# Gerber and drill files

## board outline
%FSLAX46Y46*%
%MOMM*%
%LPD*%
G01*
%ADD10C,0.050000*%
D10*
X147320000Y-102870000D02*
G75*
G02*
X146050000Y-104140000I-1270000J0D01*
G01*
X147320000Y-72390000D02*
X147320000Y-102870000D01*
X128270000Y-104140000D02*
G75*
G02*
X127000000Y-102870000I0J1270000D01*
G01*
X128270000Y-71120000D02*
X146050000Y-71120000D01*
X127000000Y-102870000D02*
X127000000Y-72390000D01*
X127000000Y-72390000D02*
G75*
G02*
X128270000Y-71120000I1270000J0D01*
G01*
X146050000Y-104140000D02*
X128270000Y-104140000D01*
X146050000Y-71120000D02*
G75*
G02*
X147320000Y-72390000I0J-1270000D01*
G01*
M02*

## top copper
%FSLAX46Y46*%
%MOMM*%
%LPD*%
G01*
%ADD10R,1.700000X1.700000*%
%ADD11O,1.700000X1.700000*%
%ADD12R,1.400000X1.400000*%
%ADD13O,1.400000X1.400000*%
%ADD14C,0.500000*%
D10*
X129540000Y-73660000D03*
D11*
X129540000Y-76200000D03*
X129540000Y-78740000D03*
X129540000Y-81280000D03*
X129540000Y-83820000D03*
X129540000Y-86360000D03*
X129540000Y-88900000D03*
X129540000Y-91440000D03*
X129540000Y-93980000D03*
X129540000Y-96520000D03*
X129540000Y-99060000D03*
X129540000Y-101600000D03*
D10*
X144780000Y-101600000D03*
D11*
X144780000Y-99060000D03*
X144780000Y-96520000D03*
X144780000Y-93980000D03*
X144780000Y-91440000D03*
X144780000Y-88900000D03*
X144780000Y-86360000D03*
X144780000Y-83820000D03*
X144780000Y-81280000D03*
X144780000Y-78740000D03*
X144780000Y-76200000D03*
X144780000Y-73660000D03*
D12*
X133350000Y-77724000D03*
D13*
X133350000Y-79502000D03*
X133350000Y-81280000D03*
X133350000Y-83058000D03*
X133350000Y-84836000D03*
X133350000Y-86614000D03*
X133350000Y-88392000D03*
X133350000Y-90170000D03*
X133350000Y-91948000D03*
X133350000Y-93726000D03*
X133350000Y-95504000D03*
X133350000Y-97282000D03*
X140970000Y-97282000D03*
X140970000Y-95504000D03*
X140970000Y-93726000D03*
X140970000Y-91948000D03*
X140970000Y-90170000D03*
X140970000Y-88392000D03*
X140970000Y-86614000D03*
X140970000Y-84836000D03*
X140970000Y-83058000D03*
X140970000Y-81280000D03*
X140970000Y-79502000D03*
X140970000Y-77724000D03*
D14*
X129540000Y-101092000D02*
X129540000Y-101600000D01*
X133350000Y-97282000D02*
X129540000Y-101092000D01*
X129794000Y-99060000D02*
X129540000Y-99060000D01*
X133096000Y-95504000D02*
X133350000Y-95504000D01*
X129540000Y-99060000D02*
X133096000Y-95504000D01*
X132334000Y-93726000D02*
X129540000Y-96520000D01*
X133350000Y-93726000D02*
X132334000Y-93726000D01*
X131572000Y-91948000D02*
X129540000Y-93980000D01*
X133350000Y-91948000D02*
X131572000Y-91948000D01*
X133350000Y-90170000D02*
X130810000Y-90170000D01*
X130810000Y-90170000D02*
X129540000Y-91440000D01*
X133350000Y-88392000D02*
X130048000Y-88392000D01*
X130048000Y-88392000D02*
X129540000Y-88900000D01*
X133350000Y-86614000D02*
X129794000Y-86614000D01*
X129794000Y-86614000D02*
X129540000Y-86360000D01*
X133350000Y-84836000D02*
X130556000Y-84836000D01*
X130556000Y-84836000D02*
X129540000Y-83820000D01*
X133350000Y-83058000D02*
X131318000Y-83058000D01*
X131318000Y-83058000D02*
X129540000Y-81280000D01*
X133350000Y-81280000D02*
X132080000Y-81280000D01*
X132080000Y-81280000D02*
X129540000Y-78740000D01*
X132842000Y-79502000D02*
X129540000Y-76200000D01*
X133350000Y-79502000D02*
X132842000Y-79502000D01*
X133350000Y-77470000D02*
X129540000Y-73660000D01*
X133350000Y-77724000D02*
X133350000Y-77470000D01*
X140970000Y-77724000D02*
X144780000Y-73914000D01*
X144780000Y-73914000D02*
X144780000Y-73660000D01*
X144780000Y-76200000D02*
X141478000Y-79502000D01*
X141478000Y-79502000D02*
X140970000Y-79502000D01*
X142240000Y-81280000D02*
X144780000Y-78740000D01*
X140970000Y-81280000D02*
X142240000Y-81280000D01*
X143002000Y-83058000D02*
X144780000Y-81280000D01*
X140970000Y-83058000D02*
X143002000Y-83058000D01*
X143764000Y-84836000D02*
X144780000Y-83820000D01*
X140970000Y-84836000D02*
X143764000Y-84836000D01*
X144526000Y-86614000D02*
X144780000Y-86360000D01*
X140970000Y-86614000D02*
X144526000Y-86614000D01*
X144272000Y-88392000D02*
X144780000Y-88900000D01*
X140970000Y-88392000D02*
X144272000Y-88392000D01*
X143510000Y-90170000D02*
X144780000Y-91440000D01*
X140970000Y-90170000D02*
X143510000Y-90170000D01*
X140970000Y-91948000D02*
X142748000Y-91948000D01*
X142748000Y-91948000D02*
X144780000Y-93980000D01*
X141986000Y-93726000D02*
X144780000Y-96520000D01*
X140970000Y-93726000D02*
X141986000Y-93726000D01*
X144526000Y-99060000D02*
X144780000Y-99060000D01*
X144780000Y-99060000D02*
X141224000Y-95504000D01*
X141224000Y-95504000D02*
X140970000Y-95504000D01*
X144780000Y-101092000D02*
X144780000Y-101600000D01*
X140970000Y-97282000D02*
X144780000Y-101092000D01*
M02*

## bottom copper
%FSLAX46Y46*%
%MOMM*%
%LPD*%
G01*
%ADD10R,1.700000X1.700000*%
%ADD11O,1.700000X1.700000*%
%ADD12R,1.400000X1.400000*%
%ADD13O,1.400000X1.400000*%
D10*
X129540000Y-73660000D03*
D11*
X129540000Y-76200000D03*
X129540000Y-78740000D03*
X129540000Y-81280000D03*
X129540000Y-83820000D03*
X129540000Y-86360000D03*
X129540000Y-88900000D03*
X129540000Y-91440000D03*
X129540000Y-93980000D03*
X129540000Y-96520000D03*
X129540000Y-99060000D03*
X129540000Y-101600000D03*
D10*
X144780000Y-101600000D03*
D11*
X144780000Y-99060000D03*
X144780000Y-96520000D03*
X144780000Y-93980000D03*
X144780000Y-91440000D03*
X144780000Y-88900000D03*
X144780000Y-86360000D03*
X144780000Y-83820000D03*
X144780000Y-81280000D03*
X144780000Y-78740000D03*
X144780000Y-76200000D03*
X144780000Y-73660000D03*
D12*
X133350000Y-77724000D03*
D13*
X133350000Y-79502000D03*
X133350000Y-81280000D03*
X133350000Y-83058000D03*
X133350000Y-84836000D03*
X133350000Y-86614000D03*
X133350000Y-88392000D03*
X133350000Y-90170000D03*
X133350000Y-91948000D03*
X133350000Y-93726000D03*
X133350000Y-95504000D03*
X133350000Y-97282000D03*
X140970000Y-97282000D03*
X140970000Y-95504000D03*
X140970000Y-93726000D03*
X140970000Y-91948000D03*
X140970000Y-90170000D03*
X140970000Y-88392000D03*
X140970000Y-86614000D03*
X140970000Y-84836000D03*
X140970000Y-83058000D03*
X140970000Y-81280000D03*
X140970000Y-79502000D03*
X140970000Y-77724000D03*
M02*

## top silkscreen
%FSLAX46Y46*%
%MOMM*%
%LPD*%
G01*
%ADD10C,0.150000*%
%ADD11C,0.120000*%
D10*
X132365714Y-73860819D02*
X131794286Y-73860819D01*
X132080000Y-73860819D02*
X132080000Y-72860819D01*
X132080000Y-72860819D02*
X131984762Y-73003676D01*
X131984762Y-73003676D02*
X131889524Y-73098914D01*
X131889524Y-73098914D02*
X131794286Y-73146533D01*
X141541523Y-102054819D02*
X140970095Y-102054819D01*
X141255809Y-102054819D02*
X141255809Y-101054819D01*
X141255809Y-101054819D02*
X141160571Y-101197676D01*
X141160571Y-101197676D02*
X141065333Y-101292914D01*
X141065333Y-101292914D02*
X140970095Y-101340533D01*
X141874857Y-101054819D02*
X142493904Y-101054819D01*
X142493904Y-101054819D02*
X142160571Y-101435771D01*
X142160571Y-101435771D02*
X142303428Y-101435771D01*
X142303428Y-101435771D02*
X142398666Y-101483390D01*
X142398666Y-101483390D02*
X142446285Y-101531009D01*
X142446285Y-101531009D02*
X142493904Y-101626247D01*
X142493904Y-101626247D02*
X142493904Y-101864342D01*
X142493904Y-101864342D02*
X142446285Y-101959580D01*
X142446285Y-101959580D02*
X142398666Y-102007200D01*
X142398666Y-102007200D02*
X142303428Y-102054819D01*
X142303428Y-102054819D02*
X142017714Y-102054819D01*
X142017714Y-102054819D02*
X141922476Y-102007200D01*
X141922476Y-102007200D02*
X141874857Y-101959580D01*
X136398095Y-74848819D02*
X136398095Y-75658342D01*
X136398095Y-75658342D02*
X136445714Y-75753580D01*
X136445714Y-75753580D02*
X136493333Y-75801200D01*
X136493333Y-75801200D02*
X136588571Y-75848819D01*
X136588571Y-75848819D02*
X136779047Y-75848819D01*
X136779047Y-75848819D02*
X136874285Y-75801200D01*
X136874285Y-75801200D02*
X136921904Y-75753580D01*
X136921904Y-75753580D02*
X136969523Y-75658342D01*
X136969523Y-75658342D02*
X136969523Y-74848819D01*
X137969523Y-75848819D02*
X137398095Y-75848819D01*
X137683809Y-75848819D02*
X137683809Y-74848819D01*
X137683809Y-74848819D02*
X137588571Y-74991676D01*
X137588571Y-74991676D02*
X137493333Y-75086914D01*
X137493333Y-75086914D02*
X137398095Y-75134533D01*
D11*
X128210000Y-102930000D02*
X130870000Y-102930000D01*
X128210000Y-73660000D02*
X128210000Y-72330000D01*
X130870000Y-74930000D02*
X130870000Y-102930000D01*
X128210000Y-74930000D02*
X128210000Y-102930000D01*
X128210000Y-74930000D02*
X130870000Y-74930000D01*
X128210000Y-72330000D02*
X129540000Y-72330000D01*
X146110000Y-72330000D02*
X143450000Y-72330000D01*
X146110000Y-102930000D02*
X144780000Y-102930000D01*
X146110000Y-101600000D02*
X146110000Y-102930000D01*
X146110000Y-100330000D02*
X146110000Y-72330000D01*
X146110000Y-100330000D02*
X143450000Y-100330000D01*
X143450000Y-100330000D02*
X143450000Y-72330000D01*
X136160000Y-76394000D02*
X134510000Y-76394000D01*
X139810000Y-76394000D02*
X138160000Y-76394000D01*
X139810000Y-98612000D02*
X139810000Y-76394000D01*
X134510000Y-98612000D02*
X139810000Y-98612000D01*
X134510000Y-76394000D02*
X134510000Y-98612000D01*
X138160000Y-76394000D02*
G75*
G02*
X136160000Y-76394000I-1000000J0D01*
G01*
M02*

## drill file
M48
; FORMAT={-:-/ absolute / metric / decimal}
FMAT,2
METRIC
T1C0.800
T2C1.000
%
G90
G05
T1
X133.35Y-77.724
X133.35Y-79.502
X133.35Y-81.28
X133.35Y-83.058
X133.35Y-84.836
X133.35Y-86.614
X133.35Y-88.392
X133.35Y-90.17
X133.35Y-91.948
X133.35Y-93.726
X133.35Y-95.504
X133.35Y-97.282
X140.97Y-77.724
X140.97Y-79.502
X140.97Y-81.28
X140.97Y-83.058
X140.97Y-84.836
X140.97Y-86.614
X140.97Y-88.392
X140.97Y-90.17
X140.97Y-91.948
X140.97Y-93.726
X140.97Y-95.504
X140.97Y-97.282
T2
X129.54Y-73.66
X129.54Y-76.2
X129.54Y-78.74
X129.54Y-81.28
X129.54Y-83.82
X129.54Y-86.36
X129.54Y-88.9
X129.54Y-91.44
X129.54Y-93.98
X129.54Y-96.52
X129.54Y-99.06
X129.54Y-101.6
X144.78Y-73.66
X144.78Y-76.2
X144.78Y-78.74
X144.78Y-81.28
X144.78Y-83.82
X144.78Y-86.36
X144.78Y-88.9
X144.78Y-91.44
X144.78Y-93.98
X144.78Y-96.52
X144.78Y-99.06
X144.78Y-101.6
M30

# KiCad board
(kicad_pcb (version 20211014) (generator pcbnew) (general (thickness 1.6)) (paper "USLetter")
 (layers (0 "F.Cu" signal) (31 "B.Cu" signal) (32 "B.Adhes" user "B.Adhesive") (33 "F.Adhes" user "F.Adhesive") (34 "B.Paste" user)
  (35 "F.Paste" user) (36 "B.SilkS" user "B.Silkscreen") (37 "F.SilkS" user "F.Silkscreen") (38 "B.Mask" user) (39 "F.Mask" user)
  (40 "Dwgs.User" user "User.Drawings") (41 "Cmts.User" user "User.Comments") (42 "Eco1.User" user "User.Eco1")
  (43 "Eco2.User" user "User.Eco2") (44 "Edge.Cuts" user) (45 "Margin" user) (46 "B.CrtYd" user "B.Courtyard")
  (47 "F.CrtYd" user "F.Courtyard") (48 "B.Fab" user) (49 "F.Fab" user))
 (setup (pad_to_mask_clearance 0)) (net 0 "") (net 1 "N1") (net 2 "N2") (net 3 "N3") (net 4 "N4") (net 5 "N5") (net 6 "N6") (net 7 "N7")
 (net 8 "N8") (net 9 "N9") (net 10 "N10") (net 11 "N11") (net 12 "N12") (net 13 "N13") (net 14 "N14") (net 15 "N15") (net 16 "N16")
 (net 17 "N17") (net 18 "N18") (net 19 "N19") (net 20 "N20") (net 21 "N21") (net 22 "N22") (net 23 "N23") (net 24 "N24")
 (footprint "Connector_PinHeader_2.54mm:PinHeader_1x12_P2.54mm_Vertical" (layer "F.Cu") (at 129.54 73.66)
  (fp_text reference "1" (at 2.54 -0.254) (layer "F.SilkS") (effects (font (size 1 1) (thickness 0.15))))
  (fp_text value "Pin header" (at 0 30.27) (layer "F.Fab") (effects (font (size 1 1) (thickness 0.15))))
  (fp_line (start -1.33 29.27) (end 1.33 29.27) (layer "F.SilkS") (width 0.12))
  (fp_line (start -1.33 0) (end -1.33 -1.33) (layer "F.SilkS") (width 0.12))
  (fp_line (start 1.33 1.27) (end 1.33 29.27) (layer "F.SilkS") (width 0.12))
  (fp_line (start -1.33 1.27) (end -1.33 29.27) (layer "F.SilkS") (width 0.12))
  (fp_line (start -1.33 1.27) (end 1.33 1.27) (layer "F.SilkS") (width 0.12))
  (fp_line (start -1.33 -1.33) (end 0 -1.33) (layer "F.SilkS") (width 0.12))
  (pad "1" thru_hole rect locked (at 0 0) (size 1.7 1.7) (drill 1) (layers *.Cu *.Mask) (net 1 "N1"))
  (pad "2" thru_hole oval locked (at 0 2.54) (size 1.7 1.7) (drill 1) (layers *.Cu *.Mask) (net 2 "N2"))
  (pad "3" thru_hole oval locked (at 0 5.08) (size 1.7 1.7) (drill 1) (layers *.Cu *.Mask) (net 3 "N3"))
  (pad "4" thru_hole oval locked (at 0 7.62) (size 1.7 1.7) (drill 1) (layers *.Cu *.Mask) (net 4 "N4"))
  (pad "5" thru_hole oval locked (at 0 10.16) (size 1.7 1.7) (drill 1) (layers *.Cu *.Mask) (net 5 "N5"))
  (pad "6" thru_hole oval locked (at 0 12.7) (size 1.7 1.7) (drill 1) (layers *.Cu *.Mask) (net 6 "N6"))
  (pad "7" thru_hole oval locked (at 0 15.24) (size 1.7 1.7) (drill 1) (layers *.Cu *.Mask) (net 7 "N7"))
  (pad "8" thru_hole oval locked (at 0 17.78) (size 1.7 1.7) (drill 1) (layers *.Cu *.Mask) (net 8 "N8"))
  (pad "9" thru_hole oval locked (at 0 20.32) (size 1.7 1.7) (drill 1) (layers *.Cu *.Mask) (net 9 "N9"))
  (pad "10" thru_hole oval locked (at 0 22.86) (size 1.7 1.7) (drill 1) (layers *.Cu *.Mask) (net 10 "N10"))
  (pad "11" thru_hole oval locked (at 0 25.4) (size 1.7 1.7) (drill 1) (layers *.Cu *.Mask) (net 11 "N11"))
  (pad "12" thru_hole oval locked (at 0 27.94) (size 1.7 1.7) (drill 1) (layers *.Cu *.Mask) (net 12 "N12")))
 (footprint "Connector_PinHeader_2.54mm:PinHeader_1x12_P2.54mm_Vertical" (layer "F.Cu") (at 144.78 101.6 180)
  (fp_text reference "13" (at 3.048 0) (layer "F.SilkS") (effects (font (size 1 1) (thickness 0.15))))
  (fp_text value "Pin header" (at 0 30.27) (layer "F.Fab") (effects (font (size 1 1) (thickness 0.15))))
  (fp_line (start -1.33 29.27) (end 1.33 29.27) (layer "F.SilkS") (width 0.12))
  (fp_line (start -1.33 -1.33) (end 0 -1.33) (layer "F.SilkS") (width 0.12))
  (fp_line (start -1.33 0) (end -1.33 -1.33) (layer "F.SilkS") (width 0.12))
  (fp_line (start -1.33 1.27) (end -1.33 29.27) (layer "F.SilkS") (width 0.12))
  (fp_line (start -1.33 1.27) (end 1.33 1.27) (layer "F.SilkS") (width 0.12))
  (fp_line (start 1.33 1.27) (end 1.33 29.27) (layer "F.SilkS") (width 0.12))
  (pad "1" thru_hole rect locked (at 0 0 180) (size 1.7 1.7) (drill 1) (layers *.Cu *.Mask) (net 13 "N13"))
  (pad "2" thru_hole oval locked (at 0 2.54 180) (size 1.7 1.7) (drill 1) (layers *.Cu *.Mask) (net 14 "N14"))
  (pad "3" thru_hole oval locked (at 0 5.08 180) (size 1.7 1.7) (drill 1) (layers *.Cu *.Mask) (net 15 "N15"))
  (pad "4" thru_hole oval locked (at 0 7.62 180) (size 1.7 1.7) (drill 1) (layers *.Cu *.Mask) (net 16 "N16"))
  (pad "5" thru_hole oval locked (at 0 10.16 180) (size 1.7 1.7) (drill 1) (layers *.Cu *.Mask) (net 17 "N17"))
  (pad "6" thru_hole oval locked (at 0 12.7 180) (size 1.7 1.7) (drill 1) (layers *.Cu *.Mask) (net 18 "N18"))
  (pad "7" thru_hole oval locked (at 0 15.24 180) (size 1.7 1.7) (drill 1) (layers *.Cu *.Mask) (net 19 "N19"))
  (pad "8" thru_hole oval locked (at 0 17.78 180) (size 1.7 1.7) (drill 1) (layers *.Cu *.Mask) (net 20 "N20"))
  (pad "9" thru_hole oval locked (at 0 20.32 180) (size 1.7 1.7) (drill 1) (layers *.Cu *.Mask) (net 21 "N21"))
  (pad "10" thru_hole oval locked (at 0 22.86 180) (size 1.7 1.7) (drill 1) (layers *.Cu *.Mask) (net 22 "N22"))
  (pad "11" thru_hole oval locked (at 0 25.4 180) (size 1.7 1.7) (drill 1) (layers *.Cu *.Mask) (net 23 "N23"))
  (pad "12" thru_hole oval locked (at 0 27.94 180) (size 1.7 1.7) (drill 1) (layers *.Cu *.Mask) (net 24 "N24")))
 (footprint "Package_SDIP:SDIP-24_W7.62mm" (layer "F.Cu") (at 133.35 77.724)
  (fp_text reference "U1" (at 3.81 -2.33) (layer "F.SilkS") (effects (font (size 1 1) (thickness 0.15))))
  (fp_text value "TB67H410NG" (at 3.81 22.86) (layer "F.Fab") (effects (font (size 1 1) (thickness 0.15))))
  (fp_line (start 2.81 -1.33) (end 1.16 -1.33) (layer "F.SilkS") (width 0.12))
  (fp_line (start 6.46 -1.33) (end 4.81 -1.33) (layer "F.SilkS") (width 0.12))
  (fp_line (start 6.46 20.888) (end 6.46 -1.33) (layer "F.SilkS") (width 0.12))
  (fp_line (start 1.16 20.888) (end 6.46 20.888) (layer "F.SilkS") (width 0.12))
  (fp_line (start 1.16 -1.33) (end 1.16 20.888) (layer "F.SilkS") (width 0.12))
  (fp_arc (start 4.81 -1.33) (mid 3.81 -0.33) (end 2.81 -1.33) (layer "F.SilkS") (width 0.12))
  (pad "1" thru_hole rect locked (at 0 0) (size 1.4 1.4) (drill 0.8) (layers *.Cu *.Mask) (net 1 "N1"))
  (pad "2" thru_hole oval locked (at 0 1.778) (size 1.4 1.4) (drill 0.8) (layers *.Cu *.Mask) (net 2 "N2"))
  (pad "3" thru_hole oval locked (at 0 3.556) (size 1.4 1.4) (drill 0.8) (layers *.Cu *.Mask) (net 3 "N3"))
  (pad "4" thru_hole oval locked (at 0 5.334) (size 1.4 1.4) (drill 0.8) (layers *.Cu *.Mask) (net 4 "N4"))
  (pad "5" thru_hole oval locked (at 0 7.112) (size 1.4 1.4) (drill 0.8) (layers *.Cu *.Mask) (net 5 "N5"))
  (pad "6" thru_hole oval locked (at 0 8.89) (size 1.4 1.4) (drill 0.8) (layers *.Cu *.Mask) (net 6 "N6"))
  (pad "7" thru_hole oval locked (at 0 10.668) (size 1.4 1.4) (drill 0.8) (layers *.Cu *.Mask) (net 7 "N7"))
  (pad "8" thru_hole oval locked (at 0 12.446) (size 1.4 1.4) (drill 0.8) (layers *.Cu *.Mask) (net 8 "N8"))
  (pad "9" thru_hole oval locked (at 0 14.224) (size 1.4 1.4) (drill 0.8) (layers *.Cu *.Mask) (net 9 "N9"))
  (pad "10" thru_hole oval locked (at 0 16.002) (size 1.4 1.4) (drill 0.8) (layers *.Cu *.Mask) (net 10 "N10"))
  (pad "11" thru_hole oval locked (at 0 17.78) (size 1.4 1.4) (drill 0.8) (layers *.Cu *.Mask) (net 11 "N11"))
  (pad "12" thru_hole oval locked (at 0 19.558) (size 1.4 1.4) (drill 0.8) (layers *.Cu *.Mask) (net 12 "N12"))
  (pad "13" thru_hole oval locked (at 7.62 19.558) (size 1.4 1.4) (drill 0.8) (layers *.Cu *.Mask) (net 13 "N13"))
  (pad "14" thru_hole oval locked (at 7.62 17.78) (size 1.4 1.4) (drill 0.8) (layers *.Cu *.Mask) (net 14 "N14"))
  (pad "15" thru_hole oval locked (at 7.62 16.002) (size 1.4 1.4) (drill 0.8) (layers *.Cu *.Mask) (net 15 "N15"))
  (pad "16" thru_hole oval locked (at 7.62 14.224) (size 1.4 1.4) (drill 0.8) (layers *.Cu *.Mask) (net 16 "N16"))
  (pad "17" thru_hole oval locked (at 7.62 12.446) (size 1.4 1.4) (drill 0.8) (layers *.Cu *.Mask) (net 17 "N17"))
  (pad "18" thru_hole oval locked (at 7.62 10.668) (size 1.4 1.4) (drill 0.8) (layers *.Cu *.Mask) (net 18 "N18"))
  (pad "19" thru_hole oval locked (at 7.62 8.89) (size 1.4 1.4) (drill 0.8) (layers *.Cu *.Mask) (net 19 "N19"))
  (pad "20" thru_hole oval locked (at 7.62 7.112) (size 1.4 1.4) (drill 0.8) (layers *.Cu *.Mask) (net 20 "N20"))
  (pad "21" thru_hole oval locked (at 7.62 5.334) (size 1.4 1.4) (drill 0.8) (layers *.Cu *.Mask) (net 21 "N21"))
  (pad "22" thru_hole oval locked (at 7.62 3.556) (size 1.4 1.4) (drill 0.8) (layers *.Cu *.Mask) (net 22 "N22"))
  (pad "23" thru_hole oval locked (at 7.62 1.778) (size 1.4 1.4) (drill 0.8) (layers *.Cu *.Mask) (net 23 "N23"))
  (pad "24" thru_hole oval locked (at 7.62 0) (size 1.4 1.4) (drill 0.8) (layers *.Cu *.Mask) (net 24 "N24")))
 (gr_arc (start 147.32 102.87) (mid 146.948026 103.768026) (end 146.05 104.14) (layer "Edge.Cuts") (width 0.05))
 (gr_line (start 147.32 72.39) (end 147.32 102.87) (layer "Edge.Cuts") (width 0.05))
 (gr_arc (start 128.27 104.14) (mid 127.371974 103.768026) (end 127 102.87) (layer "Edge.Cuts") (width 0.05))
 (gr_line (start 128.27 71.12) (end 146.05 71.12) (layer "Edge.Cuts") (width 0.05))
 (gr_line (start 127 102.87) (end 127 72.39) (layer "Edge.Cuts") (width 0.05))
 (gr_arc (start 127 72.39) (mid 127.371974 71.491974) (end 128.27 71.12) (layer "Edge.Cuts") (width 0.05))
 (gr_line (start 146.05 104.14) (end 128.27 104.14) (layer "Edge.Cuts") (width 0.05))
 (gr_arc (start 146.05 71.12) (mid 146.948026 71.491974) (end 147.32 72.39) (layer "Edge.Cuts") (width 0.05))
 (segment (start 129.54 101.092) (end 129.54 101.6) (width 0.5) (layer "F.Cu") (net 12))
 (segment (start 133.35 97.282) (end 129.54 101.092) (width 0.5) (layer "F.Cu") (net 12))
 (segment (start 129.794 99.06) (end 129.54 99.06) (width 0.5) (layer "F.Cu") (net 11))
 (segment (start 133.096 95.504) (end 133.35 95.504) (width 0.5) (layer "F.Cu") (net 11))
 (segment (start 129.54 99.06) (end 133.096 95.504) (width 0.5) (layer "F.Cu") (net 11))
 (segment (start 132.334 93.726) (end 129.54 96.52) (width 0.5) (layer "F.Cu") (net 10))
 (segment (start 133.35 93.726) (end 132.334 93.726) (width 0.5) (layer "F.Cu") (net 10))
 (segment (start 131.572 91.948) (end 129.54 93.98) (width 0.5) (layer "F.Cu") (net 9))
 (segment (start 133.35 91.948) (end 131.572 91.948) (width 0.5) (layer "F.Cu") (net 9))
 (segment (start 133.35 90.17) (end 130.81 90.17) (width 0.5) (layer "F.Cu") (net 8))
 (segment (start 130.81 90.17) (end 129.54 91.44) (width 0.5) (layer "F.Cu") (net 8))
 (segment (start 133.35 88.392) (end 130.048 88.392) (width 0.5) (layer "F.Cu") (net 7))
 (segment (start 130.048 88.392) (end 129.54 88.9) (width 0.5) (layer "F.Cu") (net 7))
 (segment (start 133.35 86.614) (end 129.794 86.614) (width 0.5) (layer "F.Cu") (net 6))
 (segment (start 129.794 86.614) (end 129.54 86.36) (width 0.5) (layer "F.Cu") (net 6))
 (segment (start 133.35 84.836) (end 130.556 84.836) (width 0.5) (layer "F.Cu") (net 5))
 (segment (start 130.556 84.836) (end 129.54 83.82) (width 0.5) (layer "F.Cu") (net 5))
 (segment (start 133.35 83.058) (end 131.318 83.058) (width 0.5) (layer "F.Cu") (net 4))
 (segment (start 131.318 83.058) (end 129.54 81.28) (width 0.5) (layer "F.Cu") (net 4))
 (segment (start 133.35 81.28) (end 132.08 81.28) (width 0.5) (layer "F.Cu") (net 3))
 (segment (start 132.08 81.28) (end 129.54 78.74) (width 0.5) (layer "F.Cu") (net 3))
 (segment (start 132.842 79.502) (end 129.54 76.2) (width 0.5) (layer "F.Cu") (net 2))
 (segment (start 133.35 79.502) (end 132.842 79.502) (width 0.5) (layer "F.Cu") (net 2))
 (segment (start 133.35 77.47) (end 129.54 73.66) (width 0.5) (layer "F.Cu") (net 1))
 (segment (start 133.35 77.724) (end 133.35 77.47) (width 0.5) (layer "F.Cu") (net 1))
 (segment (start 140.97 77.724) (end 144.78 73.914) (width 0.5) (layer "F.Cu") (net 24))
 (segment (start 144.78 73.914) (end 144.78 73.66) (width 0.5) (layer "F.Cu") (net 24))
 (segment (start 144.78 76.2) (end 141.478 79.502) (width 0.5) (layer "F.Cu") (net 23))
 (segment (start 141.478 79.502) (end 140.97 79.502) (width 0.5) (layer "F.Cu") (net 23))
 (segment (start 142.24 81.28) (end 144.78 78.74) (width 0.5) (layer "F.Cu") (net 22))
 (segment (start 140.97 81.28) (end 142.24 81.28) (width 0.5) (layer "F.Cu") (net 22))
 (segment (start 143.002 83.058) (end 144.78 81.28) (width 0.5) (layer "F.Cu") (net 21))
 (segment (start 140.97 83.058) (end 143.002 83.058) (width 0.5) (layer "F.Cu") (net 21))
 (segment (start 143.764 84.836) (end 144.78 83.82) (width 0.5) (layer "F.Cu") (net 20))
 (segment (start 140.97 84.836) (end 143.764 84.836) (width 0.5) (layer "F.Cu") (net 20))
 (segment (start 144.526 86.614) (end 144.78 86.36) (width 0.5) (layer "F.Cu") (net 19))
 (segment (start 140.97 86.614) (end 144.526 86.614) (width 0.5) (layer "F.Cu") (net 19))
 (segment (start 144.272 88.392) (end 144.78 88.9) (width 0.5) (layer "F.Cu") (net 18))
 (segment (start 140.97 88.392) (end 144.272 88.392) (width 0.5) (layer "F.Cu") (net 18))
 (segment (start 143.51 90.17) (end 144.78 91.44) (width 0.5) (layer "F.Cu") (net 17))
 (segment (start 140.97 90.17) (end 143.51 90.17) (width 0.5) (layer "F.Cu") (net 17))
 (segment (start 140.97 91.948) (end 142.748 91.948) (width 0.5) (layer "F.Cu") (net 16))
 (segment (start 142.748 91.948) (end 144.78 93.98) (width 0.5) (layer "F.Cu") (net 16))
 (segment (start 141.986 93.726) (end 144.78 96.52) (width 0.5) (layer "F.Cu") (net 15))
 (segment (start 140.97 93.726) (end 141.986 93.726) (width 0.5) (layer "F.Cu") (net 15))
 (segment (start 144.526 99.06) (end 144.78 99.06) (width 0.5) (layer "F.Cu") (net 14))
 (segment (start 144.78 99.06) (end 141.224 95.504) (width 0.5) (layer "F.Cu") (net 14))
 (segment (start 141.224 95.504) (end 140.97 95.504) (width 0.5) (layer "F.Cu") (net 14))
 (segment (start 144.78 101.092) (end 144.78 101.6) (width 0.5) (layer "F.Cu") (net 13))
 (segment (start 140.97 97.282) (end 144.78 101.092) (width 0.5) (layer "F.Cu") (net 13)))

